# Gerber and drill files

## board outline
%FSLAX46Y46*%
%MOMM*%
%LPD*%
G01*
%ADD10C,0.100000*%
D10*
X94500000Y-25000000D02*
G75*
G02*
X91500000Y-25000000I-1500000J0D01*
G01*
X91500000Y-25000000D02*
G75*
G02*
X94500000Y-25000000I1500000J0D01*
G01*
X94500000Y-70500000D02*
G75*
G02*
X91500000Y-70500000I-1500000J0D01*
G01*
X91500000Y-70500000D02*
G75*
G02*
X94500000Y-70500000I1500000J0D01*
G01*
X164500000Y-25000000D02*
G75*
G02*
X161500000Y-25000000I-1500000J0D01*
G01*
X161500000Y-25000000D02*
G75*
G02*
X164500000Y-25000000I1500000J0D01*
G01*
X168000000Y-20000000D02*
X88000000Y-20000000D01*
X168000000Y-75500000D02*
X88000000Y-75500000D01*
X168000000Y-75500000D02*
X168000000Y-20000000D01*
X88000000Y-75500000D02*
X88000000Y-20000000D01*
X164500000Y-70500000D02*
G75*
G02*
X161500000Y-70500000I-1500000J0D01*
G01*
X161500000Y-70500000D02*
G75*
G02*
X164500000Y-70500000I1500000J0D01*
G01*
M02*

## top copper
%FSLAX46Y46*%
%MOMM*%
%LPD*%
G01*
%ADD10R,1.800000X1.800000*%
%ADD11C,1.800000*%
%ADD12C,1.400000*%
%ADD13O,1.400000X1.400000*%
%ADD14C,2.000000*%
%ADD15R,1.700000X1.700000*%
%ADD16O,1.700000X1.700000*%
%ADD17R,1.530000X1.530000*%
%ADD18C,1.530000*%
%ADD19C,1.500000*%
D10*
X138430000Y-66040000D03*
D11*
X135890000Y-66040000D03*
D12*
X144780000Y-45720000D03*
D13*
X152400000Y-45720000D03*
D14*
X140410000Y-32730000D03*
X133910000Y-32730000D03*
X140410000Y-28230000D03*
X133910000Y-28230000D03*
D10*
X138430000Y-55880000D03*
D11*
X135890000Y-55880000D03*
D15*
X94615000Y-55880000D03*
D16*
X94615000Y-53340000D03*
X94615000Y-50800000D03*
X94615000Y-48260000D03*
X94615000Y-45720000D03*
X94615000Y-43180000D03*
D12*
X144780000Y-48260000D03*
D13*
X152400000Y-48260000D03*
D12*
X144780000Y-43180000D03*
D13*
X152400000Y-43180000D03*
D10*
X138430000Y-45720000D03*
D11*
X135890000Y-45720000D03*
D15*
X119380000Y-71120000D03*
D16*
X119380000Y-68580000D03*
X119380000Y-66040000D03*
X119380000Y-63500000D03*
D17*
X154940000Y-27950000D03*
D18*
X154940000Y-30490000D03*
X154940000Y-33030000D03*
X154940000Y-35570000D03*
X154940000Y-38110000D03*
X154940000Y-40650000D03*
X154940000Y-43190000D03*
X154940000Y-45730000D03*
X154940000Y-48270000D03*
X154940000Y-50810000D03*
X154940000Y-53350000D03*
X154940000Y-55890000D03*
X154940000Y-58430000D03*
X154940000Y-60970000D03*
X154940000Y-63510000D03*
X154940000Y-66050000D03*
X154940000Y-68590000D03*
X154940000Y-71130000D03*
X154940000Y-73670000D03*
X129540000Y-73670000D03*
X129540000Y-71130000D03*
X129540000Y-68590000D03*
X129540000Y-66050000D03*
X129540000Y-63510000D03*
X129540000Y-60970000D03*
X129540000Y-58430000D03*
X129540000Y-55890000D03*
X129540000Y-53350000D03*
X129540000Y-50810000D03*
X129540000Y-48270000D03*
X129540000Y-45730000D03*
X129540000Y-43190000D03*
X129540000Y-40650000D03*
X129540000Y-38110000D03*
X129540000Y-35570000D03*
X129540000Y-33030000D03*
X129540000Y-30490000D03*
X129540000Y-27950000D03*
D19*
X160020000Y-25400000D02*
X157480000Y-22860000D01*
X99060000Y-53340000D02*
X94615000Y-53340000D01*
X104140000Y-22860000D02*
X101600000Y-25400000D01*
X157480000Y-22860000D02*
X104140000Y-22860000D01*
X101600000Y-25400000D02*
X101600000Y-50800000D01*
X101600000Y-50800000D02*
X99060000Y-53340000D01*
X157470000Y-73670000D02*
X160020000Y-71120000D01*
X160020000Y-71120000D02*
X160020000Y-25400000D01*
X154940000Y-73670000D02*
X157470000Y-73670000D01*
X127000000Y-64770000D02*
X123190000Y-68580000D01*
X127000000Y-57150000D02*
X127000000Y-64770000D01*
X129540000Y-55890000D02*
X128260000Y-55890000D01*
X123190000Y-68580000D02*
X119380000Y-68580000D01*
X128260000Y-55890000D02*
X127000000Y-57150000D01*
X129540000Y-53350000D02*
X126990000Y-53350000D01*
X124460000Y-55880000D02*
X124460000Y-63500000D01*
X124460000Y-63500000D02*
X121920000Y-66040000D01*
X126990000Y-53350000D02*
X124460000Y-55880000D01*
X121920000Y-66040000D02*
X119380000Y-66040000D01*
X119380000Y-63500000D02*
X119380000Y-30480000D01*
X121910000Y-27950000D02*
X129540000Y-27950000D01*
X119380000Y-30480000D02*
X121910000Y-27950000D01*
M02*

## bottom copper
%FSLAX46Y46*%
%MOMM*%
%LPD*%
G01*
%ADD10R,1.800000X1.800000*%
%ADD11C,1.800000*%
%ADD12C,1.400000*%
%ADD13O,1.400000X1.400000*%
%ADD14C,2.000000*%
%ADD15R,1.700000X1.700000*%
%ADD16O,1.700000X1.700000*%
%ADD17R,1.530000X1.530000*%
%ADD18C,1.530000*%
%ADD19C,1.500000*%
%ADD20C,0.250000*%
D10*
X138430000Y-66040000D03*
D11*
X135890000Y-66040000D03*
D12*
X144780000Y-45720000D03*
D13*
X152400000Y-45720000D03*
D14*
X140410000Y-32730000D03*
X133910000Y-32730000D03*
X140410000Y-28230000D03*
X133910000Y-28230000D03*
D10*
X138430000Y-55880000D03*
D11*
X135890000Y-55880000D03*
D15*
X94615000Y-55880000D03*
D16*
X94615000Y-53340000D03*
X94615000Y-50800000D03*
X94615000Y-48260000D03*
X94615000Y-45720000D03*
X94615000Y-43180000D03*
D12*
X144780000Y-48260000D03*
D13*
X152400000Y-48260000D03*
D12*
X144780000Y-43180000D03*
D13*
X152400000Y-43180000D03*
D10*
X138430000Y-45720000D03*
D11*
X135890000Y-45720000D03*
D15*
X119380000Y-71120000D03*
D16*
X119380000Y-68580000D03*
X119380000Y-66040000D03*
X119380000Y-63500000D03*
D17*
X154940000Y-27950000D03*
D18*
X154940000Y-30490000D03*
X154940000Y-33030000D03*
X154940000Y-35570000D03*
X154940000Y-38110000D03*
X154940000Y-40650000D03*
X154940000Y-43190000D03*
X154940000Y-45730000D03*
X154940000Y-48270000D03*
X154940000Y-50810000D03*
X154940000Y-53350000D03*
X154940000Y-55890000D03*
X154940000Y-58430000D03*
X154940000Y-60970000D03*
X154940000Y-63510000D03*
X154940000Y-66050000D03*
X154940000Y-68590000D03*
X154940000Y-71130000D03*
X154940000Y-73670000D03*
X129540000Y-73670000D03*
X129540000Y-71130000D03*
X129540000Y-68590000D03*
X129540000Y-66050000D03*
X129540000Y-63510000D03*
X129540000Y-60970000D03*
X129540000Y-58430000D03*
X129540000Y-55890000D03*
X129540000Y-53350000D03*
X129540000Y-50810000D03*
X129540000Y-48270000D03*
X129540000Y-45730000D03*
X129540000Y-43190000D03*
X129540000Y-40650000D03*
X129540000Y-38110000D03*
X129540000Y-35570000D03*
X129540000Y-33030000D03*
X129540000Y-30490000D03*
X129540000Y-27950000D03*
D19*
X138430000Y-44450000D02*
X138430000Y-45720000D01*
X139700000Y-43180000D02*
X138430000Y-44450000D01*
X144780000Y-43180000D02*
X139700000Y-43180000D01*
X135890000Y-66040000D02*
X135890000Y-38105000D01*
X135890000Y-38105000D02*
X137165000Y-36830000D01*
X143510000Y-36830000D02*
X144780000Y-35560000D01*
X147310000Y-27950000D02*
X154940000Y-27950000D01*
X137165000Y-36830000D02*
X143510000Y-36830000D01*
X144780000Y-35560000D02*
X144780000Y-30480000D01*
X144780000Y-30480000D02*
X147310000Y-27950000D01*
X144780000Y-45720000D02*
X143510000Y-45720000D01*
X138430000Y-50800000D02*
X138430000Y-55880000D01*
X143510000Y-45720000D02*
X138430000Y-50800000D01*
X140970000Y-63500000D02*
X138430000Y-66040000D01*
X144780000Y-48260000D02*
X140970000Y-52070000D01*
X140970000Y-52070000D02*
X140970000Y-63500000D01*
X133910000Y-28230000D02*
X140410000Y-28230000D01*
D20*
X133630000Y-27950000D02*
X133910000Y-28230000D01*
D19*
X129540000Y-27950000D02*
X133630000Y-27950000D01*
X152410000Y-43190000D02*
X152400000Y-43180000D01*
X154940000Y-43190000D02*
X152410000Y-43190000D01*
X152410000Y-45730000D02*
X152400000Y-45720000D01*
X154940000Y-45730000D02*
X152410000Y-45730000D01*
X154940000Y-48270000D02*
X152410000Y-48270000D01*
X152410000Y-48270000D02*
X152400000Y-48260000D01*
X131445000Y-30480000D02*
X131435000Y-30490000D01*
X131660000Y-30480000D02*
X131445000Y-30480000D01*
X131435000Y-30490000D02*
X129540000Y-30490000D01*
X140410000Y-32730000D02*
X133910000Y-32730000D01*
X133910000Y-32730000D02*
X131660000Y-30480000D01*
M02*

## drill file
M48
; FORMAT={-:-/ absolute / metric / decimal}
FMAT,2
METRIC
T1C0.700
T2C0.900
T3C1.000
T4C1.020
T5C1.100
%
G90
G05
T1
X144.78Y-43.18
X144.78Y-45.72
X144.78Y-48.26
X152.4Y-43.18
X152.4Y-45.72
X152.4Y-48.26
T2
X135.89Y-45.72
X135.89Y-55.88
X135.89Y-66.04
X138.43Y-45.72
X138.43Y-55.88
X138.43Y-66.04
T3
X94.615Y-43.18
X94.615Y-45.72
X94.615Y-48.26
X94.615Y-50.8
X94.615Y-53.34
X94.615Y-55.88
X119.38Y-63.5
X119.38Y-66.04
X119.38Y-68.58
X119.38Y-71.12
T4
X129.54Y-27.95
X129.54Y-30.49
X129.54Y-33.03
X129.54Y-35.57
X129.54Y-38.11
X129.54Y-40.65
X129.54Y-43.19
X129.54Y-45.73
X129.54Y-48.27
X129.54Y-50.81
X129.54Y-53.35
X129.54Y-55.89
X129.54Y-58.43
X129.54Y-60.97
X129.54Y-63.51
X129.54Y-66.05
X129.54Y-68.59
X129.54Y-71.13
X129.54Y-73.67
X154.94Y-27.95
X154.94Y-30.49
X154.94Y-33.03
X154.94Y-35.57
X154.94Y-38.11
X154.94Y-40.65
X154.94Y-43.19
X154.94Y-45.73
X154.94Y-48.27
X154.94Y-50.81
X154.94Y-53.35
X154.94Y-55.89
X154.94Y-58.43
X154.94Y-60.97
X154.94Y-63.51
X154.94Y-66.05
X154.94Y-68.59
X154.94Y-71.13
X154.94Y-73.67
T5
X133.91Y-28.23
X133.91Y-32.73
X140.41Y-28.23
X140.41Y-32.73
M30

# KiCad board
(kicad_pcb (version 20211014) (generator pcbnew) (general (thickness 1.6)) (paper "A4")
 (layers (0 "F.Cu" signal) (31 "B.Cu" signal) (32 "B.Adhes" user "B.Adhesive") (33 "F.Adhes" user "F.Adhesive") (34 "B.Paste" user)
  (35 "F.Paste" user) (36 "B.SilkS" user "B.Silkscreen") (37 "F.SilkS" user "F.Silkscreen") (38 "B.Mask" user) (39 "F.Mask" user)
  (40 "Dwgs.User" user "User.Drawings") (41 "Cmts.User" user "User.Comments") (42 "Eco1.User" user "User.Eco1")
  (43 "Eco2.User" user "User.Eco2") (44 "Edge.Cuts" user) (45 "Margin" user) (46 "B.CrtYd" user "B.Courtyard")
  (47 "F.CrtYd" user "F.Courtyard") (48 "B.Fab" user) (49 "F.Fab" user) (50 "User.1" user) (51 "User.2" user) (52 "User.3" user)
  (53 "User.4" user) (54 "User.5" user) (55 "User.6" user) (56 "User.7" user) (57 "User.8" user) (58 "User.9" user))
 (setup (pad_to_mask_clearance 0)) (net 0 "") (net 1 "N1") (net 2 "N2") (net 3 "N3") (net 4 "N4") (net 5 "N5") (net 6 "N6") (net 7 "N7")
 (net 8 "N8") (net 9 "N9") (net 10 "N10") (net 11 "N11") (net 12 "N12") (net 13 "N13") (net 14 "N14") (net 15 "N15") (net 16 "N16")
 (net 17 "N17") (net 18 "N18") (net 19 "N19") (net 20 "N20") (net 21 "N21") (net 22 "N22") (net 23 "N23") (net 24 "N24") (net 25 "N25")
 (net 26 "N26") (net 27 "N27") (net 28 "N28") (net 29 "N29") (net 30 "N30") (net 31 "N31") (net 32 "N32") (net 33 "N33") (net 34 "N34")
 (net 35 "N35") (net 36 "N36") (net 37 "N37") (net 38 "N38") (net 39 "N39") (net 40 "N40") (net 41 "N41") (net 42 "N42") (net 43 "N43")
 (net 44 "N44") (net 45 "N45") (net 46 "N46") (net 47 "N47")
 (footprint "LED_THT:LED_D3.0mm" (layer "F.Cu") (at 138.43 66.04 180)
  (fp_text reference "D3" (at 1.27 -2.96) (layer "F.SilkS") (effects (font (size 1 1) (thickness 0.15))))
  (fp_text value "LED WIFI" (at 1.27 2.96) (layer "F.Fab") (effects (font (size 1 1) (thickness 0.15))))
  (pad "1" thru_hole rect (at 0 0 180) (size 1.8 1.8) (drill 0.9) (layers *.Cu *.Mask) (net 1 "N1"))
  (pad "2" thru_hole circle (at 2.54 0 180) (size 1.8 1.8) (drill 0.9) (layers *.Cu *.Mask) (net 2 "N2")))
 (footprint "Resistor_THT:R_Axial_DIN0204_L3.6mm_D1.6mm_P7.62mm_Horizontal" (layer "F.Cu") (at 144.78 45.72)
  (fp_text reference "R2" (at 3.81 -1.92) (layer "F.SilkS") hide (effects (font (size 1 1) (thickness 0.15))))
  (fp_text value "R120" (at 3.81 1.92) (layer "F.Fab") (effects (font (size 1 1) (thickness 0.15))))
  (pad "1" thru_hole circle (at 0 0) (size 1.4 1.4) (drill 0.7) (layers *.Cu *.Mask) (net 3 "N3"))
  (pad "2" thru_hole oval (at 7.62 0) (size 1.4 1.4) (drill 0.7) (layers *.Cu *.Mask) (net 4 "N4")))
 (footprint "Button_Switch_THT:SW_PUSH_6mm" (layer "F.Cu") (at 140.41 32.73 180)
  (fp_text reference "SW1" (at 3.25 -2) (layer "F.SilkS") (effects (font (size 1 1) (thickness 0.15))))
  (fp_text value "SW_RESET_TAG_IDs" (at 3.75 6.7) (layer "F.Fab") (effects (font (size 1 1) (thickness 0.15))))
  (pad "1" thru_hole circle (at 0 0 270) (size 2 2) (drill 1.1) (layers *.Cu *.Mask) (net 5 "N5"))
  (pad "1" thru_hole circle (at 6.5 0 270) (size 2 2) (drill 1.1) (layers *.Cu *.Mask) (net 5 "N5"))
  (pad "2" thru_hole circle (at 0 4.5 270) (size 2 2) (drill 1.1) (layers *.Cu *.Mask) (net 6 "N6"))
  (pad "2" thru_hole circle (at 6.5 4.5 270) (size 2 2) (drill 1.1) (layers *.Cu *.Mask) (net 6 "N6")))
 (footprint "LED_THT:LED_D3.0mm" (layer "F.Cu") (at 138.43 55.88 180)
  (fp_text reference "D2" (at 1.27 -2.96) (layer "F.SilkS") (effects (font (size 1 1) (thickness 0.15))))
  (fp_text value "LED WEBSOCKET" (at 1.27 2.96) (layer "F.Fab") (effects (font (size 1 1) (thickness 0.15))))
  (pad "1" thru_hole rect (at 0 0 180) (size 1.8 1.8) (drill 0.9) (layers *.Cu *.Mask) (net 3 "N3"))
  (pad "2" thru_hole circle (at 2.54 0 180) (size 1.8 1.8) (drill 0.9) (layers *.Cu *.Mask) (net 2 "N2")))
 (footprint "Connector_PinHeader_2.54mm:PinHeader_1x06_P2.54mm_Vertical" (layer "F.Cu") (at 94.615 55.88 180)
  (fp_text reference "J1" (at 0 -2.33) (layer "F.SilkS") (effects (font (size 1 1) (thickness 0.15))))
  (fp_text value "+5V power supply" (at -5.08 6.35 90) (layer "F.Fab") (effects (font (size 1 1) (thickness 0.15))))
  (pad "1" thru_hole rect (at 0 0 180) (size 1.7 1.7) (drill 1) (layers *.Cu *.Mask) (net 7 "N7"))
  (pad "2" thru_hole oval (at 0 2.54 180) (size 1.7 1.7) (drill 1) (layers *.Cu *.Mask) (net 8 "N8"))
  (pad "3" thru_hole oval (at 0 5.08 180) (size 1.7 1.7) (drill 1) (layers *.Cu *.Mask) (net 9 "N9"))
  (pad "4" thru_hole oval (at 0 7.62 180) (size 1.7 1.7) (drill 1) (layers *.Cu *.Mask) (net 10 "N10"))
  (pad "5" thru_hole oval (at 0 10.16 180) (size 1.7 1.7) (drill 1) (layers *.Cu *.Mask) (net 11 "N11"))
  (pad "6" thru_hole oval (at 0 12.7 180) (size 1.7 1.7) (drill 1) (layers *.Cu *.Mask) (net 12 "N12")))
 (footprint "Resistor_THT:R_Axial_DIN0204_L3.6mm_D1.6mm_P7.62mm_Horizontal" (layer "F.Cu") (at 144.78 48.26)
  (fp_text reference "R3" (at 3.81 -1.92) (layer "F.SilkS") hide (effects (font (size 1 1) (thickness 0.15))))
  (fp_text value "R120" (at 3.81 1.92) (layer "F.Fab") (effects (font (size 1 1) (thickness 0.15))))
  (pad "1" thru_hole circle (at 0 0) (size 1.4 1.4) (drill 0.7) (layers *.Cu *.Mask) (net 1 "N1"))
  (pad "2" thru_hole oval (at 7.62 0) (size 1.4 1.4) (drill 0.7) (layers *.Cu *.Mask) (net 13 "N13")))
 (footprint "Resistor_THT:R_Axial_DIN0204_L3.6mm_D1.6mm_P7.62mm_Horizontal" (layer "F.Cu") (at 144.78 43.18)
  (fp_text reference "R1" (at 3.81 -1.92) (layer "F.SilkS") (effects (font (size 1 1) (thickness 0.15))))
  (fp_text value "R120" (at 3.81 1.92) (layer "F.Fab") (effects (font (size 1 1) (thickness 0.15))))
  (pad "1" thru_hole circle (at 0 0) (size 1.4 1.4) (drill 0.7) (layers *.Cu *.Mask) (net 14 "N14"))
  (pad "2" thru_hole oval (at 7.62 0) (size 1.4 1.4) (drill 0.7) (layers *.Cu *.Mask) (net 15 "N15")))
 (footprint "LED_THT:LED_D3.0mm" (layer "F.Cu") (at 138.43 45.72 180)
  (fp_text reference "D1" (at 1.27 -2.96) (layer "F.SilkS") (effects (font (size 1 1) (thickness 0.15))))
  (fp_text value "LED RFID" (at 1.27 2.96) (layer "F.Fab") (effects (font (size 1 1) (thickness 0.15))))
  (pad "1" thru_hole rect (at 0 0 180) (size 1.8 1.8) (drill 0.9) (layers *.Cu *.Mask) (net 14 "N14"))
  (pad "2" thru_hole circle (at 2.54 0 180) (size 1.8 1.8) (drill 0.9) (layers *.Cu *.Mask) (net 2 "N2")))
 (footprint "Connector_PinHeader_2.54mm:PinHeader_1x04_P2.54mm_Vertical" (layer "F.Cu") (at 119.38 71.12 180)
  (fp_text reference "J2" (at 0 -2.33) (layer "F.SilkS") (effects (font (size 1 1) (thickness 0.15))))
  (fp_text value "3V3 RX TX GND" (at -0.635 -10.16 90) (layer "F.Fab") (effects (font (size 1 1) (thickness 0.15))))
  (pad "1" thru_hole rect (at 0 0 180) (size 1.7 1.7) (drill 1) (layers *.Cu *.Mask) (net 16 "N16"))
  (pad "2" thru_hole oval (at 0 2.54 180) (size 1.7 1.7) (drill 1) (layers *.Cu *.Mask) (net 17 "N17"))
  (pad "3" thru_hole oval (at 0 5.08 180) (size 1.7 1.7) (drill 1) (layers *.Cu *.Mask) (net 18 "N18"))
  (pad "4" thru_hole oval (at 0 7.62 180) (size 1.7 1.7) (drill 1) (layers *.Cu *.Mask) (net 6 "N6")))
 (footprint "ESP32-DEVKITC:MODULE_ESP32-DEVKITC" (layer "B.Cu") (at 142.24 50.8 180)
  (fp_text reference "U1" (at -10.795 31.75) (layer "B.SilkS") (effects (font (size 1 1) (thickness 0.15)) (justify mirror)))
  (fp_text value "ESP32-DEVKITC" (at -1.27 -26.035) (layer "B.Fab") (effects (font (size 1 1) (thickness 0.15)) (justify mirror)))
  (pad "1" thru_hole rect locked (at -12.7 22.85 180) (size 1.53 1.53) (drill 1.02) (layers *.Cu *.Mask) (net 2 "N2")
   (solder_mask_margin 0.102))
  (pad "2" thru_hole circle locked (at -12.7 20.31 180) (size 1.53 1.53) (drill 1.02) (layers *.Cu *.Mask) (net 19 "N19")
   (solder_mask_margin 0.102))
  (pad "3" thru_hole circle locked (at -12.7 17.77 180) (size 1.53 1.53) (drill 1.02) (layers *.Cu *.Mask) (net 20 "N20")
   (solder_mask_margin 0.102))
  (pad "4" thru_hole circle locked (at -12.7 15.23 180) (size 1.53 1.53) (drill 1.02) (layers *.Cu *.Mask) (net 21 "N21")
   (solder_mask_margin 0.102))
  (pad "5" thru_hole circle locked (at -12.7 12.69 180) (size 1.53 1.53) (drill 1.02) (layers *.Cu *.Mask) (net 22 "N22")
   (solder_mask_margin 0.102))
  (pad "6" thru_hole circle locked (at -12.7 10.15 180) (size 1.53 1.53) (drill 1.02) (layers *.Cu *.Mask) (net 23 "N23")
   (solder_mask_margin 0.102))
  (pad "7" thru_hole circle locked (at -12.7 7.61 180) (size 1.53 1.53) (drill 1.02) (layers *.Cu *.Mask) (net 15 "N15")
   (solder_mask_margin 0.102))
  (pad "8" thru_hole circle locked (at -12.7 5.07 180) (size 1.53 1.53) (drill 1.02) (layers *.Cu *.Mask) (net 4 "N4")
   (solder_mask_margin 0.102))
  (pad "9" thru_hole circle locked (at -12.7 2.53 180) (size 1.53 1.53) (drill 1.02) (layers *.Cu *.Mask) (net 13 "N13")
   (solder_mask_margin 0.102))
  (pad "10" thru_hole circle locked (at -12.7 -0.01 180) (size 1.53 1.53) (drill 1.02) (layers *.Cu *.Mask) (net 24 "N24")
   (solder_mask_margin 0.102))
  (pad "11" thru_hole circle locked (at -12.7 -2.55 180) (size 1.53 1.53) (drill 1.02) (layers *.Cu *.Mask) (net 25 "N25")
   (solder_mask_margin 0.102))
  (pad "12" thru_hole circle locked (at -12.7 -5.09 180) (size 1.53 1.53) (drill 1.02) (layers *.Cu *.Mask) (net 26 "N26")
   (solder_mask_margin 0.102))
  (pad "13" thru_hole circle locked (at -12.7 -7.63 180) (size 1.53 1.53) (drill 1.02) (layers *.Cu *.Mask) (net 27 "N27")
   (solder_mask_margin 0.102))
  (pad "14" thru_hole circle locked (at -12.7 -10.17 180) (size 1.53 1.53) (drill 1.02) (layers *.Cu *.Mask) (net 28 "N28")
   (solder_mask_margin 0.102))
  (pad "15" thru_hole circle locked (at -12.7 -12.71 180) (size 1.53 1.53) (drill 1.02) (layers *.Cu *.Mask) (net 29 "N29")
   (solder_mask_margin 0.102))
  (pad "16" thru_hole circle locked (at -12.7 -15.25 180) (size 1.53 1.53) (drill 1.02) (layers *.Cu *.Mask) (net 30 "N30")
   (solder_mask_margin 0.102))
  (pad "17" thru_hole circle locked (at -12.7 -17.79 180) (size 1.53 1.53) (drill 1.02) (layers *.Cu *.Mask) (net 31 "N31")
   (solder_mask_margin 0.102))
  (pad "18" thru_hole circle locked (at -12.7 -20.33 180) (size 1.53 1.53) (drill 1.02) (layers *.Cu *.Mask) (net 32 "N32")
   (solder_mask_margin 0.102))
  (pad "19" thru_hole circle locked (at -12.7 -22.87 180) (size 1.53 1.53) (drill 1.02) (layers *.Cu *.Mask) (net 8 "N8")
   (solder_mask_margin 0.102))
  (pad "20" thru_hole circle locked (at 12.7 -22.87 180) (size 1.53 1.53) (drill 1.02) (layers *.Cu *.Mask) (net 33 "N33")
   (solder_mask_margin 0.102))
  (pad "21" thru_hole circle locked (at 12.7 -20.33 180) (size 1.53 1.53) (drill 1.02) (layers *.Cu *.Mask) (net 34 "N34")
   (solder_mask_margin 0.102))
  (pad "22" thru_hole circle locked (at 12.7 -17.79 180) (size 1.53 1.53) (drill 1.02) (layers *.Cu *.Mask) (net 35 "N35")
   (solder_mask_margin 0.102))
  (pad "23" thru_hole circle locked (at 12.7 -15.25 180) (size 1.53 1.53) (drill 1.02) (layers *.Cu *.Mask) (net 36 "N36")
   (solder_mask_margin 0.102))
  (pad "24" thru_hole circle locked (at 12.7 -12.71 180) (size 1.53 1.53) (drill 1.02) (layers *.Cu *.Mask) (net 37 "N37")
   (solder_mask_margin 0.102))
  (pad "25" thru_hole circle locked (at 12.7 -10.17 180) (size 1.53 1.53) (drill 1.02) (layers *.Cu *.Mask) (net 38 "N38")
   (solder_mask_margin 0.102))
  (pad "26" thru_hole circle locked (at 12.7 -7.63 180) (size 1.53 1.53) (drill 1.02) (layers *.Cu *.Mask) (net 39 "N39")
   (solder_mask_margin 0.102))
  (pad "27" thru_hole circle locked (at 12.7 -5.09 180) (size 1.53 1.53) (drill 1.02) (layers *.Cu *.Mask) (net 17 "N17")
   (solder_mask_margin 0.102))
  (pad "28" thru_hole circle locked (at 12.7 -2.55 180) (size 1.53 1.53) (drill 1.02) (layers *.Cu *.Mask) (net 18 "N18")
   (solder_mask_margin 0.102))
  (pad "29" thru_hole circle locked (at 12.7 -0.01 180) (size 1.53 1.53) (drill 1.02) (layers *.Cu *.Mask) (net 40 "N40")
   (solder_mask_margin 0.102))
  (pad "30" thru_hole circle locked (at 12.7 2.53 180) (size 1.53 1.53) (drill 1.02) (layers *.Cu *.Mask) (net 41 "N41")
   (solder_mask_margin 0.102))
  (pad "31" thru_hole circle locked (at 12.7 5.07 180) (size 1.53 1.53) (drill 1.02) (layers *.Cu *.Mask) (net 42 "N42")
   (solder_mask_margin 0.102))
  (pad "32" thru_hole circle locked (at 12.7 7.61 180) (size 1.53 1.53) (drill 1.02) (layers *.Cu *.Mask) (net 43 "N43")
   (solder_mask_margin 0.102))
  (pad "33" thru_hole circle locked (at 12.7 10.15 180) (size 1.53 1.53) (drill 1.02) (layers *.Cu *.Mask) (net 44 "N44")
   (solder_mask_margin 0.102))
  (pad "34" thru_hole circle locked (at 12.7 12.69 180) (size 1.53 1.53) (drill 1.02) (layers *.Cu *.Mask) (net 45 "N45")
   (solder_mask_margin 0.102))
  (pad "35" thru_hole circle locked (at 12.7 15.23 180) (size 1.53 1.53) (drill 1.02) (layers *.Cu *.Mask) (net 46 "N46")
   (solder_mask_margin 0.102))
  (pad "36" thru_hole circle locked (at 12.7 17.77 180) (size 1.53 1.53) (drill 1.02) (layers *.Cu *.Mask) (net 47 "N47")
   (solder_mask_margin 0.102))
  (pad "37" thru_hole circle locked (at 12.7 20.31 180) (size 1.53 1.53) (drill 1.02) (layers *.Cu *.Mask) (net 5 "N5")
   (solder_mask_margin 0.102))
  (pad "38" thru_hole circle locked (at 12.7 22.85 180) (size 1.53 1.53) (drill 1.02) (layers *.Cu *.Mask) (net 6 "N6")
   (solder_mask_margin 0.102)))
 (gr_circle (center 93 25) (end 94.5 25) (layer "Edge.Cuts") (width 0.1) (fill none))
 (gr_circle (center 93 70.5) (end 94.5 70.5) (layer "Edge.Cuts") (width 0.1) (fill none))
 (gr_circle (center 163 25) (end 164.5 25) (layer "Edge.Cuts") (width 0.1) (fill none))
 (gr_line (start 168 20) (end 88 20) (layer "Edge.Cuts") (width 0.1))
 (gr_line (start 168 75.5) (end 88 75.5) (layer "Edge.Cuts") (width 0.1))
 (gr_line (start 168 75.5) (end 168 20) (layer "Edge.Cuts") (width 0.1))
 (gr_line (start 88 75.5) (end 88 20) (layer "Edge.Cuts") (width 0.1))
 (gr_circle (center 163 70.5) (end 164.5 70.5) (layer "Edge.Cuts") (width 0.1) (fill none))
 (segment (start 138.43 44.45) (end 138.43 45.72) (width 1.5) (layer "B.Cu") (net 14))
 (segment (start 139.7 43.18) (end 138.43 44.45) (width 1.5) (layer "B.Cu") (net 14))
 (segment (start 144.78 43.18) (end 139.7 43.18) (width 1.5) (layer "B.Cu") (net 14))
 (segment (start 135.89 66.04) (end 135.89 38.105) (width 1.5) (layer "B.Cu") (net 2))
 (segment (start 135.89 38.105) (end 137.165 36.83) (width 1.5) (layer "B.Cu") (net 2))
 (segment (start 143.51 36.83) (end 144.78 35.56) (width 1.5) (layer "B.Cu") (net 2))
 (segment (start 147.31 27.95) (end 154.94 27.95) (width 1.5) (layer "B.Cu") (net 2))
 (segment (start 137.165 36.83) (end 143.51 36.83) (width 1.5) (layer "B.Cu") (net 2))
 (segment (start 144.78 35.56) (end 144.78 30.48) (width 1.5) (layer "B.Cu") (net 2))
 (segment (start 144.78 30.48) (end 147.31 27.95) (width 1.5) (layer "B.Cu") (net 2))
 (segment (start 144.78 45.72) (end 143.51 45.72) (width 1.5) (layer "B.Cu") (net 3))
 (segment (start 138.43 50.8) (end 138.43 55.88) (width 1.5) (layer "B.Cu") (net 3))
 (segment (start 143.51 45.72) (end 138.43 50.8) (width 1.5) (layer "B.Cu") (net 3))
 (segment (start 140.97 63.5) (end 138.43 66.04) (width 1.5) (layer "B.Cu") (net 1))
 (segment (start 144.78 48.26) (end 140.97 52.07) (width 1.5) (layer "B.Cu") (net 1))
 (segment (start 140.97 52.07) (end 140.97 63.5) (width 1.5) (layer "B.Cu") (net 1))
 (segment (start 160.02 25.4) (end 157.48 22.86) (width 1.5) (layer "F.Cu") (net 8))
 (segment (start 99.06 53.34) (end 94.615 53.34) (width 1.5) (layer "F.Cu") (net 8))
 (segment (start 104.14 22.86) (end 101.6 25.4) (width 1.5) (layer "F.Cu") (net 8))
 (segment (start 157.48 22.86) (end 104.14 22.86) (width 1.5) (layer "F.Cu") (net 8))
 (segment (start 101.6 25.4) (end 101.6 50.8) (width 1.5) (layer "F.Cu") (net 8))
 (segment (start 101.6 50.8) (end 99.06 53.34) (width 1.5) (layer "F.Cu") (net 8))
 (segment (start 157.47 73.67) (end 160.02 71.12) (width 1.5) (layer "F.Cu") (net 8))
 (segment (start 160.02 71.12) (end 160.02 25.4) (width 1.5) (layer "F.Cu") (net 8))
 (segment (start 154.94 73.67) (end 157.47 73.67) (width 1.5) (layer "F.Cu") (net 8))
 (segment (start 127 64.77) (end 123.19 68.58) (width 1.5) (layer "F.Cu") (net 17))
 (segment (start 127 57.15) (end 127 64.77) (width 1.5) (layer "F.Cu") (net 17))
 (segment (start 129.54 55.89) (end 128.26 55.89) (width 1.5) (layer "F.Cu") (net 17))
 (segment (start 123.19 68.58) (end 119.38 68.58) (width 1.5) (layer "F.Cu") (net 17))
 (segment (start 128.26 55.89) (end 127 57.15) (width 1.5) (layer "F.Cu") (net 17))
 (segment (start 129.54 53.35) (end 126.99 53.35) (width 1.5) (layer "F.Cu") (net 18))
 (segment (start 124.46 55.88) (end 124.46 63.5) (width 1.5) (layer "F.Cu") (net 18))
 (segment (start 124.46 63.5) (end 121.92 66.04) (width 1.5) (layer "F.Cu") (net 18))
 (segment (start 126.99 53.35) (end 124.46 55.88) (width 1.5) (layer "F.Cu") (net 18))
 (segment (start 121.92 66.04) (end 119.38 66.04) (width 1.5) (layer "F.Cu") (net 18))
 (segment (start 119.38 63.5) (end 119.38 30.48) (width 1.5) (layer "F.Cu") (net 6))
 (segment (start 121.91 27.95) (end 129.54 27.95) (width 1.5) (layer "F.Cu") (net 6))
 (segment (start 119.38 30.48) (end 121.91 27.95) (width 1.5) (layer "F.Cu") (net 6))
 (segment (start 133.91 28.23) (end 140.41 28.23) (width 1.5) (layer "B.Cu") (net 6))
 (segment (start 133.63 27.95) (end 133.91 28.23) (width 0.25) (layer "B.Cu") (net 6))
 (segment (start 129.54 27.95) (end 133.63 27.95) (width 1.5) (layer "B.Cu") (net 6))
 (segment (start 152.41 43.19) (end 152.4 43.18) (width 1.5) (layer "B.Cu") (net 15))
 (segment (start 154.94 43.19) (end 152.41 43.19) (width 1.5) (layer "B.Cu") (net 15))
 (segment (start 152.41 45.73) (end 152.4 45.72) (width 1.5) (layer "B.Cu") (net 4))
 (segment (start 154.94 45.73) (end 152.41 45.73) (width 1.5) (layer "B.Cu") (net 4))
 (segment (start 154.94 48.27) (end 152.41 48.27) (width 1.5) (layer "B.Cu") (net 13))
 (segment (start 152.41 48.27) (end 152.4 48.26) (width 1.5) (layer "B.Cu") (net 13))
 (segment (start 131.445 30.48) (end 131.435 30.49) (width 1.5) (layer "B.Cu") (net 5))
 (segment (start 131.66 30.48) (end 131.445 30.48) (width 1.5) (layer "B.Cu") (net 5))
 (segment (start 131.435 30.49) (end 129.54 30.49) (width 1.5) (layer "B.Cu") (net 5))
 (segment (start 140.41 32.73) (end 133.91 32.73) (width 1.5) (layer "B.Cu") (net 5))
 (segment (start 133.91 32.73) (end 131.66 30.48) (width 1.5) (layer "B.Cu") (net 5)))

